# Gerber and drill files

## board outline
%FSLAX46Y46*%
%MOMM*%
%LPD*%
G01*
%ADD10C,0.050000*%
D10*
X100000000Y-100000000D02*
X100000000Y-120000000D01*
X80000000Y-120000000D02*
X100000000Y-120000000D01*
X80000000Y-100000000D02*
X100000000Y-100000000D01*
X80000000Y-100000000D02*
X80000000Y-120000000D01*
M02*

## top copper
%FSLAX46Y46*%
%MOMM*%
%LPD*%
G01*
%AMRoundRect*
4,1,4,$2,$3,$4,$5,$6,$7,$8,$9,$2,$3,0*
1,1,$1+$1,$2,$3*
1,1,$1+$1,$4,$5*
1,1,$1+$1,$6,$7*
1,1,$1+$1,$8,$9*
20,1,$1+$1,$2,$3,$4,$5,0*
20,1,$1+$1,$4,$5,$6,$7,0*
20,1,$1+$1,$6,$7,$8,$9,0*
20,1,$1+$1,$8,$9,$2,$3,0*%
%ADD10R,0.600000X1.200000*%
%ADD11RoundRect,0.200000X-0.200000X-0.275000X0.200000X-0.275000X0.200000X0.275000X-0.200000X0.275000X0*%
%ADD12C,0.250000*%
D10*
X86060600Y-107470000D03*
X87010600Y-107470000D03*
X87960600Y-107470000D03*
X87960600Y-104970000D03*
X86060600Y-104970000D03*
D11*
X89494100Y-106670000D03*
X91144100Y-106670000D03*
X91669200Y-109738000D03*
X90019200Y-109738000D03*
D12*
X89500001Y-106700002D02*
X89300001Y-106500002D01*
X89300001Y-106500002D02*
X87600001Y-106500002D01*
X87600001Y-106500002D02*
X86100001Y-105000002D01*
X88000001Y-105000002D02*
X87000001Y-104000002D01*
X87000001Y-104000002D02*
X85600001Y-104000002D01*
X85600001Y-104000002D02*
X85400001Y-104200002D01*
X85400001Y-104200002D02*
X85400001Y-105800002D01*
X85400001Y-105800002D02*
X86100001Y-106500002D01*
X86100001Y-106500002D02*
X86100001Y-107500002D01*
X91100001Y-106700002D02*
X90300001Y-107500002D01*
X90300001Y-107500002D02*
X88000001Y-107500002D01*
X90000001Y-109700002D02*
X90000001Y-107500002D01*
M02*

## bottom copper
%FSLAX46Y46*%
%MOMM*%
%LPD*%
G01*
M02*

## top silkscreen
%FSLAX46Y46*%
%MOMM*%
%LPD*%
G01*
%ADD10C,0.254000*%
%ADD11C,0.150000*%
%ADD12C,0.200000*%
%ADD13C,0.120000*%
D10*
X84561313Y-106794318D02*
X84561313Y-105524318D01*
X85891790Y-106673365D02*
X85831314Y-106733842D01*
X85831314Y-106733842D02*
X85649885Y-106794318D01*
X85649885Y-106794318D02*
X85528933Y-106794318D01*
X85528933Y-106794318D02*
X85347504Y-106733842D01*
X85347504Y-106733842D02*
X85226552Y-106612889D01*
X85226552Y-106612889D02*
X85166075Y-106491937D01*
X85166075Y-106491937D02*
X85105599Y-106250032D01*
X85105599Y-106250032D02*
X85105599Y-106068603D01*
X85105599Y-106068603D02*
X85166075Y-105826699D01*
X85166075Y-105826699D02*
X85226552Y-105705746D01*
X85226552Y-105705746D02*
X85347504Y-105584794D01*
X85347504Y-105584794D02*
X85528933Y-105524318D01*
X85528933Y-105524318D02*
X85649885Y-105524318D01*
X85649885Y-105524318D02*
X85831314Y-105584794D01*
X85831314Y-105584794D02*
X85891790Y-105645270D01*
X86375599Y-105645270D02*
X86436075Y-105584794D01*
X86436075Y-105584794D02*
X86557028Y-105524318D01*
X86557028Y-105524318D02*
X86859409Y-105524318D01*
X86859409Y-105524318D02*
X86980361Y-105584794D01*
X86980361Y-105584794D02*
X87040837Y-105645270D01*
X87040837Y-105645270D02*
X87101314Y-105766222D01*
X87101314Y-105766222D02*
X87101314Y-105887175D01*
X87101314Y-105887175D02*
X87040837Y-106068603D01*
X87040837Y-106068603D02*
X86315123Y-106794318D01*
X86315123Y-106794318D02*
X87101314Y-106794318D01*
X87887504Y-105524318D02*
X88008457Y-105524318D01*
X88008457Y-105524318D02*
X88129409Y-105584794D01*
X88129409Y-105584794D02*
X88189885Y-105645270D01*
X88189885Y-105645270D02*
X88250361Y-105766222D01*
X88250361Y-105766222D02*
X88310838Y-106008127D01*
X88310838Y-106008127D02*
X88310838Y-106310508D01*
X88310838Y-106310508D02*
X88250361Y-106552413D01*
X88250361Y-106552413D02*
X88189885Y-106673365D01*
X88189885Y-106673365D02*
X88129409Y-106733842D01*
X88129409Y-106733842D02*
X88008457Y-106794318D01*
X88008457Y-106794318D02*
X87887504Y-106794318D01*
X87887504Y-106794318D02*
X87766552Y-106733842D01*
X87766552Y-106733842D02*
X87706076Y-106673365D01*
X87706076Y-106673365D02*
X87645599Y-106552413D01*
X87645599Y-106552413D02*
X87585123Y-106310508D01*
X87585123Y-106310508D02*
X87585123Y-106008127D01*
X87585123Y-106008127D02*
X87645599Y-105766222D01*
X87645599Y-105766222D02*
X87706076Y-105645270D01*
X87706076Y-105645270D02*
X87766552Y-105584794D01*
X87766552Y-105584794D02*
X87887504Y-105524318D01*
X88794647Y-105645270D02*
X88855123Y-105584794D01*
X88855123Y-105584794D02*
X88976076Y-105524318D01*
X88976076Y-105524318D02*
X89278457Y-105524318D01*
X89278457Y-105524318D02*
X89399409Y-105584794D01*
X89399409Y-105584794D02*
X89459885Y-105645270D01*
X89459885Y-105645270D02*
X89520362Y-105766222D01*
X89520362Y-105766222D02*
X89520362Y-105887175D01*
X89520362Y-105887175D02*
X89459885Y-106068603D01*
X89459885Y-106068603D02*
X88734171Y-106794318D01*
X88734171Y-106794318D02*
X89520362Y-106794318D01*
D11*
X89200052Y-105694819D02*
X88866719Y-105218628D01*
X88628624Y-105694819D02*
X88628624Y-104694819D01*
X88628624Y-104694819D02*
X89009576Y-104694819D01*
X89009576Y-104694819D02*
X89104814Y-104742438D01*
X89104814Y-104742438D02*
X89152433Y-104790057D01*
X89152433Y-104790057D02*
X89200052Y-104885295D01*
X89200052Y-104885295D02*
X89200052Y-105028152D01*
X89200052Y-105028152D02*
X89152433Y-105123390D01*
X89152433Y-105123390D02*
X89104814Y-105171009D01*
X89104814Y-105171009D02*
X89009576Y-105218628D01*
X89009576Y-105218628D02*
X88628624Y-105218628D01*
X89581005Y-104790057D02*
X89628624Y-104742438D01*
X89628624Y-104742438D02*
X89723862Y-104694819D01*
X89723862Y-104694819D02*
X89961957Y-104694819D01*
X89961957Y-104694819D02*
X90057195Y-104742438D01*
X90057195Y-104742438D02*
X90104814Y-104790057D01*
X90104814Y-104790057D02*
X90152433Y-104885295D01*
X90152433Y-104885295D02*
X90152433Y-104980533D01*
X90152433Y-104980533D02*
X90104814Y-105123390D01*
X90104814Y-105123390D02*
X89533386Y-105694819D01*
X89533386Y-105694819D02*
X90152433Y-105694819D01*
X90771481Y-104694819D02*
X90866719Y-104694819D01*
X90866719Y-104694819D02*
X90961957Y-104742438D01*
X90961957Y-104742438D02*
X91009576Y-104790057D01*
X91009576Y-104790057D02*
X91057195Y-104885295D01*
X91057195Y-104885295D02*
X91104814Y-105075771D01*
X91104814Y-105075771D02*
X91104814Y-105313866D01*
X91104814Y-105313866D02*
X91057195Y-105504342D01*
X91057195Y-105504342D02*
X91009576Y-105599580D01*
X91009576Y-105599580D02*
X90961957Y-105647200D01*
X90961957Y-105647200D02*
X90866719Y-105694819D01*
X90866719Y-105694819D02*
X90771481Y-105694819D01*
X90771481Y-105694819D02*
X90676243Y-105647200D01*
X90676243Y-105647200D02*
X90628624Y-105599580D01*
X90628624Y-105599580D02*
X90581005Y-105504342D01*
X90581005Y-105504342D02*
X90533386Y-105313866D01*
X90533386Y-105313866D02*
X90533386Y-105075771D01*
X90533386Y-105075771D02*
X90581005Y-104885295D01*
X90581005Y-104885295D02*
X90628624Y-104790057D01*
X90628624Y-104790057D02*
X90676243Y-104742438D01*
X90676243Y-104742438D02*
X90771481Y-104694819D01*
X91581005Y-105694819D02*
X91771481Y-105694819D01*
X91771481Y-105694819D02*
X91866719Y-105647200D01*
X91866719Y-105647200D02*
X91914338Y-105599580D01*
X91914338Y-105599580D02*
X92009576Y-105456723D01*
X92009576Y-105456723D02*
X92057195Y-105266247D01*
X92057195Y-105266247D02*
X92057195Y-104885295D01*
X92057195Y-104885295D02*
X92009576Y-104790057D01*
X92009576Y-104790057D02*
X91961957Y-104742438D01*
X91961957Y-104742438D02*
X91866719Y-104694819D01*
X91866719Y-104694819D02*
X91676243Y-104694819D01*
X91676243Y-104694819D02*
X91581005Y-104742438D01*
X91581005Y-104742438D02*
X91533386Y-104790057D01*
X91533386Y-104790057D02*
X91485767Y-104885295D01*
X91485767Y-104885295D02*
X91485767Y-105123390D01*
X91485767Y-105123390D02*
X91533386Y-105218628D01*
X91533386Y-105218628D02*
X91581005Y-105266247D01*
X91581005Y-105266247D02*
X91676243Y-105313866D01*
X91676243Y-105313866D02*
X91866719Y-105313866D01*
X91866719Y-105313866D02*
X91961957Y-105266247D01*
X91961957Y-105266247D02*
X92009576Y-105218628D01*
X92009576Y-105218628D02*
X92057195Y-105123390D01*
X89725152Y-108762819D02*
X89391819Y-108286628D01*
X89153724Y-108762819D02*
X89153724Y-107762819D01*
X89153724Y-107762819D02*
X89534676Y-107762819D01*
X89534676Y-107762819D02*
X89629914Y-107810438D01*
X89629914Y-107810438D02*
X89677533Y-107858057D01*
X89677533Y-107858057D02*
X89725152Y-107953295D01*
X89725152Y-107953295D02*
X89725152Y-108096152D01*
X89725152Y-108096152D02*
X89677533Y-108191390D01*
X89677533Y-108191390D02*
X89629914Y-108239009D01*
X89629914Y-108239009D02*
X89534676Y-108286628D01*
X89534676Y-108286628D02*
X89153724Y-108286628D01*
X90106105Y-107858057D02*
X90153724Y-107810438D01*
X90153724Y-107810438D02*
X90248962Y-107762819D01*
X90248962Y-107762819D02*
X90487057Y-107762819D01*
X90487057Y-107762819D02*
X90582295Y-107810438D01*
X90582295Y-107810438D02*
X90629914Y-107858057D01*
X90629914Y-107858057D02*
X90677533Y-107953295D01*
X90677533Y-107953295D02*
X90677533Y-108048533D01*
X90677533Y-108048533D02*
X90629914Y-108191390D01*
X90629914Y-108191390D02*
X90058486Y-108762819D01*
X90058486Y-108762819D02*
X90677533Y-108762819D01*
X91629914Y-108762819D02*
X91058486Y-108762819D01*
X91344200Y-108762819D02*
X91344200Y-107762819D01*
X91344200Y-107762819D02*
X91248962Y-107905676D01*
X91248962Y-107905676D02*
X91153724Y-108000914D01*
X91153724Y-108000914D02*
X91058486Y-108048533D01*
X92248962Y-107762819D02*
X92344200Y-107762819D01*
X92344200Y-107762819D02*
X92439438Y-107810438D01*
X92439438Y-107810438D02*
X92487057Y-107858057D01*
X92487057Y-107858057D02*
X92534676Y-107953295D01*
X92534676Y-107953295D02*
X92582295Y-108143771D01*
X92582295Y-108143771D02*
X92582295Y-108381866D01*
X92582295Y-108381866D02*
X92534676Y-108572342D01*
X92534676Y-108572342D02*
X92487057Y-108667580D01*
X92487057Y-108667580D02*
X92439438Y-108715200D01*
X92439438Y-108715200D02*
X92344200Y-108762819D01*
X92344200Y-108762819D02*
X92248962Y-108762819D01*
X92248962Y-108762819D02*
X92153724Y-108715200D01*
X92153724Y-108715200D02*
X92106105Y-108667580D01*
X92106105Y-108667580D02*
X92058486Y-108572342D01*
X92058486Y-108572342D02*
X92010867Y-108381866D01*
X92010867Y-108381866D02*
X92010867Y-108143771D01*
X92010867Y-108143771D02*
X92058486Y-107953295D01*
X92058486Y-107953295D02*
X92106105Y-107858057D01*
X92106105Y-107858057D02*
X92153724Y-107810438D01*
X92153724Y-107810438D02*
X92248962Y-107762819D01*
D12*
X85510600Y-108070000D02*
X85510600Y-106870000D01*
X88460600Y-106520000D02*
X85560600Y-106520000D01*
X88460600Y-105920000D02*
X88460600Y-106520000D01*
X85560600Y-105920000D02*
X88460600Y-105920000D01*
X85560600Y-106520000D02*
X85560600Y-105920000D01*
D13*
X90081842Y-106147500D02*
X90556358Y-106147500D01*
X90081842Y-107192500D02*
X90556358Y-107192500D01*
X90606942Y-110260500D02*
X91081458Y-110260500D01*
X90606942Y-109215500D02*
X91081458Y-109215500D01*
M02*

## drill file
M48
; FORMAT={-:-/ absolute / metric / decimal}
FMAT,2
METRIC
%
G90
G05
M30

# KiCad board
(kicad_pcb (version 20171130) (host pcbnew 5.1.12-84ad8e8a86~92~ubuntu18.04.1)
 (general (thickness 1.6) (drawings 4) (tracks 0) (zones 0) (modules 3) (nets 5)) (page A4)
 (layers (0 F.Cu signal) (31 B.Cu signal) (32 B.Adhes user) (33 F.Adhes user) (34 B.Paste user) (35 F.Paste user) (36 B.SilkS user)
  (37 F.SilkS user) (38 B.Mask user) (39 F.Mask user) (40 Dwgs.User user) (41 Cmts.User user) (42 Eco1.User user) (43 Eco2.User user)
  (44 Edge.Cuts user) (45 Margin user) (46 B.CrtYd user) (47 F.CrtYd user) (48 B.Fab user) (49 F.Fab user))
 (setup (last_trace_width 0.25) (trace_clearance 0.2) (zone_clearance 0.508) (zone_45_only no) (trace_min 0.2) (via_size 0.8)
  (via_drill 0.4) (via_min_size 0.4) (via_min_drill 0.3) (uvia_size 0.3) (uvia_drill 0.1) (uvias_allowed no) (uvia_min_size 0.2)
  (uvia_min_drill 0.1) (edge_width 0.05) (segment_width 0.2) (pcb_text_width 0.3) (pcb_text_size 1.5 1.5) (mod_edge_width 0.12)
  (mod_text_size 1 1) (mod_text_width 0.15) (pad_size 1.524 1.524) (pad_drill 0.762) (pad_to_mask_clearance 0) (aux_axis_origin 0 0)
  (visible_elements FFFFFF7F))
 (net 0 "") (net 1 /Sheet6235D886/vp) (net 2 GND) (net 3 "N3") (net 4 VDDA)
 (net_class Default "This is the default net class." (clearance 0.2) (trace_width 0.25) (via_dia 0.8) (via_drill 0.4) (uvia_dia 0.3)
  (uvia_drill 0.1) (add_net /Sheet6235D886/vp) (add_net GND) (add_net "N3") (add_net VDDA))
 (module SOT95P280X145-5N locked (layer F.Cu) (at 87.010600 106.220000 90.000000)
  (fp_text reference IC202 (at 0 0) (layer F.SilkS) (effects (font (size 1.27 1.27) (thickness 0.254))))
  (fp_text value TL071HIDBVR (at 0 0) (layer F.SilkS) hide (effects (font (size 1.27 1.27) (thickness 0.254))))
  (fp_line (start -1.85 -1.5) (end -0.65 -1.5) (layer F.SilkS) (width 0.2))
  (fp_line (start -0.3 1.45) (end -0.3 -1.45) (layer F.SilkS) (width 0.2))
  (fp_line (start 0.3 1.45) (end -0.3 1.45) (layer F.SilkS) (width 0.2))
  (fp_line (start 0.3 -1.45) (end 0.3 1.45) (layer F.SilkS) (width 0.2))
  (fp_line (start -0.3 -1.45) (end 0.3 -1.45) (layer F.SilkS) (width 0.2))
  (pad 1 smd rect (at -1.25 -0.95 180.000000) (size 0.6 1.2) (layers F.Cu F.Mask F.Paste) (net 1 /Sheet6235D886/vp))
  (pad 2 smd rect (at -1.25 0 180.000000) (size 0.6 1.2) (layers F.Cu F.Mask F.Paste) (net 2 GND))
  (pad 3 smd rect (at -1.25 0.95 180.000000) (size 0.6 1.2) (layers F.Cu F.Mask F.Paste) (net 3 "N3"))
  (pad 4 smd rect (at 1.25 0.95 180.000000) (size 0.6 1.2) (layers F.Cu F.Mask F.Paste) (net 1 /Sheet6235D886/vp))
  (pad 5 smd rect (at 1.25 -0.95 180.000000) (size 0.6 1.2) (layers F.Cu F.Mask F.Paste) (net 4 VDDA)))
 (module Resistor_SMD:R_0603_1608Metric (layer F.Cu) (at 90.319100 106.670000)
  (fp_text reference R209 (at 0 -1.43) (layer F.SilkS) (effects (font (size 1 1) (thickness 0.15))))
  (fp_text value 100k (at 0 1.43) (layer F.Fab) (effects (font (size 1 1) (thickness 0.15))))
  (fp_line (start -0.237258 -0.5225) (end 0.237258 -0.5225) (layer F.SilkS) (width 0.12))
  (fp_line (start -0.237258 0.5225) (end 0.237258 0.5225) (layer F.SilkS) (width 0.12))
  (pad 1 smd roundrect (at -0.825 0) (size 0.8 0.95) (layers F.Cu F.Mask F.Paste) (roundrect_rratio 0.25) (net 4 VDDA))
  (pad 2 smd roundrect (at 0.825 0) (size 0.8 0.95) (layers F.Cu F.Mask F.Paste) (roundrect_rratio 0.25) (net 3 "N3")))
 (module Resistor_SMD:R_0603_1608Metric (layer F.Cu) (at 90.844200 109.738000)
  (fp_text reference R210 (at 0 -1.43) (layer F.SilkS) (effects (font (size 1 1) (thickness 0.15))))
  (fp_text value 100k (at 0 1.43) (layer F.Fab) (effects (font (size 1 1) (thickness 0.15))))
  (fp_line (start -0.237258 0.5225) (end 0.237258 0.5225) (layer F.SilkS) (width 0.12))
  (fp_line (start -0.237258 -0.5225) (end 0.237258 -0.5225) (layer F.SilkS) (width 0.12))
  (pad 2 smd roundrect (at 0.825 0) (size 0.8 0.95) (layers F.Cu F.Mask F.Paste) (roundrect_rratio 0.25) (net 2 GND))
  (pad 1 smd roundrect (at -0.825 0) (size 0.8 0.95) (layers F.Cu F.Mask F.Paste) (roundrect_rratio 0.25) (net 3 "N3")))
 (gr_line (start 100 100) (end 100 120) (layer Edge.Cuts) (width 0.05))
 (gr_line (start 80 120) (end 100 120) (layer Edge.Cuts) (width 0.05))
 (gr_line (start 80 100) (end 100 100) (layer Edge.Cuts) (width 0.05))
 (gr_line (start 80 100) (end 80 120) (layer Edge.Cuts) (width 0.05))
 (segment (start 89.500001 106.700002) (end 89.300001 106.500002) (width 0.250000) (layer F.Cu) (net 4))
 (segment (start 89.300001 106.500002) (end 87.600001 106.500002) (width 0.250000) (layer F.Cu) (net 4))
 (segment (start 87.600001 106.500002) (end 86.100001 105.000002) (width 0.250000) (layer F.Cu) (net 4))
 (segment (start 88.000001 105.000002) (end 87.000001 104.000002) (width 0.250000) (layer F.Cu) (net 1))
 (segment (start 87.000001 104.000002) (end 85.600001 104.000002) (width 0.250000) (layer F.Cu) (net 1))
 (segment (start 85.600001 104.000002) (end 85.400001 104.200002) (width 0.250000) (layer F.Cu) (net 1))
 (segment (start 85.400001 104.200002) (end 85.400001 105.800002) (width 0.250000) (layer F.Cu) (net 1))
 (segment (start 85.400001 105.800002) (end 86.100001 106.500002) (width 0.250000) (layer F.Cu) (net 1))
 (segment (start 86.100001 106.500002) (end 86.100001 107.500002) (width 0.250000) (layer F.Cu) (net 1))
 (segment (start 91.100001 106.700002) (end 90.300001 107.500002) (width 0.250000) (layer F.Cu) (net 3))
 (segment (start 90.300001 107.500002) (end 88.000001 107.500002) (width 0.250000) (layer F.Cu) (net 3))
 (segment (start 90.000001 109.700002) (end 90.000001 107.500002) (width 0.250000) (layer F.Cu) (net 3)))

